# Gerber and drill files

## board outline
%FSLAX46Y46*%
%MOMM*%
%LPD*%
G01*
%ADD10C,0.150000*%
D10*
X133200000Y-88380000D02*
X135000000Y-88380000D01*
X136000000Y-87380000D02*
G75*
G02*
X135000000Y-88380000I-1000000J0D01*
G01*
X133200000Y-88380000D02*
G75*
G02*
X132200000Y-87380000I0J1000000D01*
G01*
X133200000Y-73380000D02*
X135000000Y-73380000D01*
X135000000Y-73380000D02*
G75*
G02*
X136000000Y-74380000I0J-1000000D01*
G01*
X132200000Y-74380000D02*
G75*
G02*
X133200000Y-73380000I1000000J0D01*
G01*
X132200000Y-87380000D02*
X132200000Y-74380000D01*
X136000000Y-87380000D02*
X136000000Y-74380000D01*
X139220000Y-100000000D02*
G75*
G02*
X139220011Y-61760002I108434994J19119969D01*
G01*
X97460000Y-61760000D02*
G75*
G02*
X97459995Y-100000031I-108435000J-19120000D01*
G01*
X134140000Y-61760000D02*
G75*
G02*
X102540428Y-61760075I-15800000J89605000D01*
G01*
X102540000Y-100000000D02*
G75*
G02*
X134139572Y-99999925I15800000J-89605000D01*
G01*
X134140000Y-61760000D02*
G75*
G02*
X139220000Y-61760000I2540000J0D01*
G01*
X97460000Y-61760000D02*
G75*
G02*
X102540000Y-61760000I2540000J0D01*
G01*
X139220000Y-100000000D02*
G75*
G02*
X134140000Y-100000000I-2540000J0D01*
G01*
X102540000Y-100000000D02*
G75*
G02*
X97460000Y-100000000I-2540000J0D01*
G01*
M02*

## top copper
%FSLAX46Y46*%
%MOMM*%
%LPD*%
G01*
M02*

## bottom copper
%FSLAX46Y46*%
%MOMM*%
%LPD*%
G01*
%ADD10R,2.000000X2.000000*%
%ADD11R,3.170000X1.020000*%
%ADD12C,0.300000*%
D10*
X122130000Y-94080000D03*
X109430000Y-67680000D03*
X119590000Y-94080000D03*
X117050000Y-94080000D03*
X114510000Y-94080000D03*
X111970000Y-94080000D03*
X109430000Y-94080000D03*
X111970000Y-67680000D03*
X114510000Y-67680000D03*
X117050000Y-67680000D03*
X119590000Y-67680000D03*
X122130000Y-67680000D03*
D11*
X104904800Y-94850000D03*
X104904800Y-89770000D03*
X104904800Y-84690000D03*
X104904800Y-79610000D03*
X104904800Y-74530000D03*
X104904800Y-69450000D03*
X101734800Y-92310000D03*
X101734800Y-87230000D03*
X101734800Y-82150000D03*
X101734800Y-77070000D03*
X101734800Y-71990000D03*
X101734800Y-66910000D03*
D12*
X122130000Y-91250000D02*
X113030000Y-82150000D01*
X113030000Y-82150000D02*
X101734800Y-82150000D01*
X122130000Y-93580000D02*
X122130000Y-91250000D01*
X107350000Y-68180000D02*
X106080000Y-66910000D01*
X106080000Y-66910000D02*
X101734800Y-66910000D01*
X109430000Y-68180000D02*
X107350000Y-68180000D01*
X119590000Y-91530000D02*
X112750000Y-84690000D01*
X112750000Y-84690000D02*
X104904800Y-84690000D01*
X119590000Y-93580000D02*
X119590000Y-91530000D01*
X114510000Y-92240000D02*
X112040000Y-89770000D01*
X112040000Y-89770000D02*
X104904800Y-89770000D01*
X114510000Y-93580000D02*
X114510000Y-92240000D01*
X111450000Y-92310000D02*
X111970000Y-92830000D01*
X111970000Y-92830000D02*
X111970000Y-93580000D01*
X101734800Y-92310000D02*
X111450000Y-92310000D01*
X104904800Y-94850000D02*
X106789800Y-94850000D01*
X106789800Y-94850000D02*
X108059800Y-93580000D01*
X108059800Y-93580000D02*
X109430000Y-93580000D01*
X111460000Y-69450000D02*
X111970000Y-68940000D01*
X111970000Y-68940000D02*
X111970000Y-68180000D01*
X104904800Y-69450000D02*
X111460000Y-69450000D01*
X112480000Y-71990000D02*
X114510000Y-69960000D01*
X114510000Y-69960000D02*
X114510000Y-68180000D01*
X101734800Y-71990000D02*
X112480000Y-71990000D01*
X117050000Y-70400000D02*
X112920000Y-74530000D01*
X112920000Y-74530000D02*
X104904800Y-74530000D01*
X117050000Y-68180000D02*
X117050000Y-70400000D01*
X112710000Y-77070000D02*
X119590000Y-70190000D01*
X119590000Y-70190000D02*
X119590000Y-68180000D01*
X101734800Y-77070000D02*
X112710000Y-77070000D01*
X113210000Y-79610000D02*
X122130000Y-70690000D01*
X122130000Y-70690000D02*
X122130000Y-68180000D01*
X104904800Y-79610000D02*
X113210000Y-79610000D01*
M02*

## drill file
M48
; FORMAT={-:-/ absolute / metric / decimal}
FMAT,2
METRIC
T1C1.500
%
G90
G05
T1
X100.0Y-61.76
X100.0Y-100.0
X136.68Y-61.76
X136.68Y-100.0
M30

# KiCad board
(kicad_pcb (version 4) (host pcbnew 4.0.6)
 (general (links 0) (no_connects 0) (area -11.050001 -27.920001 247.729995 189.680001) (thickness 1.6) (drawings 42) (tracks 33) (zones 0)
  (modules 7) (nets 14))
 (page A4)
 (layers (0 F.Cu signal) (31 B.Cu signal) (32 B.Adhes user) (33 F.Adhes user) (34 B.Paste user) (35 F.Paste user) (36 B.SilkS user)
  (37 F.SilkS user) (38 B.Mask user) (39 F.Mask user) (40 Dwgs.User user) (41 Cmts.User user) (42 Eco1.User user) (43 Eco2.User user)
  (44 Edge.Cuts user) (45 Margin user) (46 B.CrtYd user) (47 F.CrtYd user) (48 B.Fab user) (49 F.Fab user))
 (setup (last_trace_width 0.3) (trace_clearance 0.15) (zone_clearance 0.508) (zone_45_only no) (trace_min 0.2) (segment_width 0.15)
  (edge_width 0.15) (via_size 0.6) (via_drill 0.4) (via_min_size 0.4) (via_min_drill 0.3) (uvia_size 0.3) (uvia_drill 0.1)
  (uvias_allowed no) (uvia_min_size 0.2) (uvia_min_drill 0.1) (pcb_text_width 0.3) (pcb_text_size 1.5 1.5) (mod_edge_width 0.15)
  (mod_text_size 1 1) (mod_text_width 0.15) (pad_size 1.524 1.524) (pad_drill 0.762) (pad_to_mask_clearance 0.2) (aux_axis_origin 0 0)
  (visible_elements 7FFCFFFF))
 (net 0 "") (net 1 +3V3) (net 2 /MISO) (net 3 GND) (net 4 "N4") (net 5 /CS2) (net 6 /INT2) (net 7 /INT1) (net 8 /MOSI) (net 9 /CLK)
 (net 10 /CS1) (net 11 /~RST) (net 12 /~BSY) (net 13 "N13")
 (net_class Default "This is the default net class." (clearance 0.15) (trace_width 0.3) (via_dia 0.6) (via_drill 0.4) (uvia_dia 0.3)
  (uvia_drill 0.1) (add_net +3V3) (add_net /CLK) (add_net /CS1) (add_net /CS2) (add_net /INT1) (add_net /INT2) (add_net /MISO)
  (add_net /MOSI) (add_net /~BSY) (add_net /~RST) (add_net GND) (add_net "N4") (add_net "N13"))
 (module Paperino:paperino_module (layer B.Cu) (at 118.73 80.88 90)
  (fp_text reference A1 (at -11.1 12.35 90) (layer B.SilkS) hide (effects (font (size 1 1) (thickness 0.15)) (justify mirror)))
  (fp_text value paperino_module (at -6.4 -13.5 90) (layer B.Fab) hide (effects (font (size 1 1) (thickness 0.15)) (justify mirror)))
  (pad 1 smd rect (at -12.7 3.4 90) (size 2 2) (drill (offset -0.5 0)) (layers B.Cu B.Paste B.Mask) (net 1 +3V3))
  (pad 7 smd rect (at 12.7 -9.3 90) (size 2 2) (drill (offset 0.5 0)) (layers B.Cu B.Paste B.Mask) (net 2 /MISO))
  (pad 2 smd rect (at -12.7 0.86 90) (size 2 2) (drill (offset -0.5 0)) (layers B.Cu B.Paste B.Mask) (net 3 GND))
  (pad 3 smd rect (at -12.7 -1.68 90) (size 2 2) (drill (offset -0.5 0)) (layers B.Cu B.Paste B.Mask) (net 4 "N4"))
  (pad 4 smd rect (at -12.7 -4.22 90) (size 2 2) (drill (offset -0.5 0)) (layers B.Cu B.Paste B.Mask) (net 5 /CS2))
  (pad 5 smd rect (at -12.7 -6.76 90) (size 2 2) (drill (offset -0.5 0)) (layers B.Cu B.Paste B.Mask) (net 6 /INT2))
  (pad 6 smd rect (at -12.7 -9.3 90) (size 2 2) (drill (offset -0.5 0)) (layers B.Cu B.Paste B.Mask) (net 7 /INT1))
  (pad 8 smd rect (at 12.7 -6.76 90) (size 2 2) (drill (offset 0.5 0)) (layers B.Cu B.Paste B.Mask) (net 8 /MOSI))
  (pad 9 smd rect (at 12.7 -4.22 90) (size 2 2) (drill (offset 0.5 0)) (layers B.Cu B.Paste B.Mask) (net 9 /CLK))
  (pad 10 smd rect (at 12.7 -1.68 90) (size 2 2) (drill (offset 0.5 0)) (layers B.Cu B.Paste B.Mask) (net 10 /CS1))
  (pad 11 smd rect (at 12.7 0.86 90) (size 2 2) (drill (offset 0.5 0)) (layers B.Cu B.Paste B.Mask) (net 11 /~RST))
  (pad 12 smd rect (at 12.7 3.4 90) (size 2 2) (drill (offset 0.5 0)) (layers B.Cu B.Paste B.Mask) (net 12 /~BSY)))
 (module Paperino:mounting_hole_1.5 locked (layer F.Cu) (at 100 100)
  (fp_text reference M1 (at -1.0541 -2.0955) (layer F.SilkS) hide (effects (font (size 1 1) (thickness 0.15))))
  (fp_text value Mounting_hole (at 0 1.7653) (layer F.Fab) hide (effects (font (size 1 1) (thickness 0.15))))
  (pad "" np_thru_hole circle (at 0 0) (size 1.5 1.5) (drill 1.5) (layers *.Cu *.Mask)))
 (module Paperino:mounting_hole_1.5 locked (layer F.Cu) (at 136.68 100)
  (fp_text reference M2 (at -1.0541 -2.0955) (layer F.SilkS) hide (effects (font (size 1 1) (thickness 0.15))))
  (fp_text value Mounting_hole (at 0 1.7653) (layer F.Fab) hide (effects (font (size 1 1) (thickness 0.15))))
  (pad "" np_thru_hole circle (at 0 0) (size 1.5 1.5) (drill 1.5) (layers *.Cu *.Mask)))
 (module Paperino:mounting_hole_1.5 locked (layer F.Cu) (at 100 61.76)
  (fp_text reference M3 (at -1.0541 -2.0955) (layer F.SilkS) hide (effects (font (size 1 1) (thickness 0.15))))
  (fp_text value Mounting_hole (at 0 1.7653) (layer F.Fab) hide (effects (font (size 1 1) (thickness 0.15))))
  (pad "" np_thru_hole circle (at 0 0) (size 1.5 1.5) (drill 1.5) (layers *.Cu *.Mask)))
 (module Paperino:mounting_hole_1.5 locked (layer F.Cu) (at 136.68 61.76)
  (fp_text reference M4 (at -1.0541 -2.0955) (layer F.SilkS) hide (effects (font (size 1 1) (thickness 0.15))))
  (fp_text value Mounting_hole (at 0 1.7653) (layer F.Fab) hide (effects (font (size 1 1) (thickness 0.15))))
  (pad "" np_thru_hole circle (at 0 0) (size 1.5 1.5) (drill 1.5) (layers *.Cu *.Mask)))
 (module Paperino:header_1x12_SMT (layer B.Cu) (at 103.32 80.88 90)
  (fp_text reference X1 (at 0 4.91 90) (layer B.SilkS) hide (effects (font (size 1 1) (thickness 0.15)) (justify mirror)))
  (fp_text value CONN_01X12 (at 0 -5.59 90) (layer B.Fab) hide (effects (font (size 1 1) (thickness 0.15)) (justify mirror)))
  (pad 1 smd rect (at -13.97 1.5848 90) (size 1.02 3.17) (layers B.Cu B.Paste B.Mask) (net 7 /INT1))
  (pad 3 smd rect (at -8.89 1.5848 90) (size 1.02 3.17) (layers B.Cu B.Paste B.Mask) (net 5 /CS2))
  (pad 5 smd rect (at -3.81 1.5848 90) (size 1.02 3.17) (layers B.Cu B.Paste B.Mask) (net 3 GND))
  (pad 7 smd rect (at 1.27 1.5848 90) (size 1.02 3.17) (layers B.Cu B.Paste B.Mask) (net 12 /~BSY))
  (pad 9 smd rect (at 6.35 1.5848 90) (size 1.02 3.17) (layers B.Cu B.Paste B.Mask) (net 10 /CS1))
  (pad 11 smd rect (at 11.43 1.5848 90) (size 1.02 3.17) (layers B.Cu B.Paste B.Mask) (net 8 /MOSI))
  (pad 2 smd rect (at -11.43 -1.5852 90) (size 1.02 3.17) (layers B.Cu B.Paste B.Mask) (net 6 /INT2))
  (pad 4 smd rect (at -6.35 -1.5852 90) (size 1.02 3.17) (layers B.Cu B.Paste B.Mask) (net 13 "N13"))
  (pad 6 smd rect (at -1.27 -1.5852 90) (size 1.02 3.17) (layers B.Cu B.Paste B.Mask) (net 1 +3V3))
  (pad 8 smd rect (at 3.81 -1.5852 90) (size 1.02 3.17) (layers B.Cu B.Paste B.Mask) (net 11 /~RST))
  (pad 10 smd rect (at 8.89 -1.5852 90) (size 1.02 3.17) (layers B.Cu B.Paste B.Mask) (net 9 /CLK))
  (pad 12 smd rect (at 13.97 -1.5852 90) (size 1.02 3.17) (layers B.Cu B.Paste B.Mask) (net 2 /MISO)))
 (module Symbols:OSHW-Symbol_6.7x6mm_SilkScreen (layer F.Cu) (at 133.66 67.9 90)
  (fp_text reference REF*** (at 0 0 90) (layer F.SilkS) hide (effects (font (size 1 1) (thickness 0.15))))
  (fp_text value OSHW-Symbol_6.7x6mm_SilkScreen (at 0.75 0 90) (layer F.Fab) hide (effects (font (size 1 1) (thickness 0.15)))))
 (gr_line (start 133.2 88.38) (end 135 88.38) (layer Edge.Cuts) (width 0.15))
 (gr_arc (start 135 87.38) (end 136 87.38) (angle 90) (layer Edge.Cuts) (width 0.15))
 (gr_arc (start 133.2 87.38) (end 133.2 88.38) (angle 90) (layer Edge.Cuts) (width 0.15))
 (gr_line (start 133.2 73.38) (end 135 73.38) (layer Edge.Cuts) (width 0.15))
 (gr_arc (start 135 74.38) (end 135 73.38) (angle 90) (layer Edge.Cuts) (width 0.15))
 (gr_arc (start 133.2 74.38) (end 132.2 74.38) (angle 90) (layer Edge.Cuts) (width 0.15))
 (gr_line (start 132.2 87.38) (end 132.2 74.38) (layer Edge.Cuts) (width 0.15))
 (gr_line (start 136 87.38) (end 136 74.38) (layer Edge.Cuts) (width 0.15))
 (gr_arc (start 247.654994 80.880031) (end 139.22 100) (angle 19.9999845) (layer Edge.Cuts) (width 0.15))
 (gr_arc (start -10.975 80.88) (end 97.46 61.76) (angle 20) (layer Edge.Cuts) (width 0.15))
 (gr_arc (start 118.34 -27.845) (end 134.14 61.76) (angle 20) (layer Edge.Cuts) (width 0.15))
 (gr_arc (start 118.34 189.605) (end 102.54 100) (angle 20) (layer Edge.Cuts) (width 0.15))
 (gr_arc (start 136.68 61.76) (end 134.14 61.76) (angle 180) (layer Edge.Cuts) (width 0.15))
 (gr_arc (start 100 61.76) (end 97.46 61.76) (angle 180) (layer Edge.Cuts) (width 0.15))
 (gr_arc (start 136.68 100) (end 139.22 100) (angle 180) (layer Edge.Cuts) (width 0.15))
 (gr_arc (start 100 100) (end 102.54 100) (angle 180) (layer Edge.Cuts) (width 0.15))
 (segment (start 122.13 91.25) (end 113.03 82.15) (width 0.3) (layer B.Cu) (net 1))
 (segment (start 113.03 82.15) (end 101.7348 82.15) (width 0.3) (layer B.Cu) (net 1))
 (segment (start 122.13 93.58) (end 122.13 91.25) (width 0.3) (layer B.Cu) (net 1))
 (segment (start 107.35 68.18) (end 106.08 66.91) (width 0.3) (layer B.Cu) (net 2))
 (segment (start 106.08 66.91) (end 101.7348 66.91) (width 0.3) (layer B.Cu) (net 2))
 (segment (start 109.43 68.18) (end 107.35 68.18) (width 0.3) (layer B.Cu) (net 2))
 (segment (start 119.59 91.53) (end 112.75 84.69) (width 0.3) (layer B.Cu) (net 3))
 (segment (start 112.75 84.69) (end 104.9048 84.69) (width 0.3) (layer B.Cu) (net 3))
 (segment (start 119.59 93.58) (end 119.59 91.53) (width 0.3) (layer B.Cu) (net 3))
 (segment (start 114.51 92.24) (end 112.04 89.77) (width 0.3) (layer B.Cu) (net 5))
 (segment (start 112.04 89.77) (end 104.9048 89.77) (width 0.3) (layer B.Cu) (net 5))
 (segment (start 114.51 93.58) (end 114.51 92.24) (width 0.3) (layer B.Cu) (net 5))
 (segment (start 111.45 92.31) (end 111.97 92.83) (width 0.3) (layer B.Cu) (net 6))
 (segment (start 111.97 92.83) (end 111.97 93.58) (width 0.3) (layer B.Cu) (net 6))
 (segment (start 101.7348 92.31) (end 111.45 92.31) (width 0.3) (layer B.Cu) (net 6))
 (segment (start 104.9048 94.85) (end 106.7898 94.85) (width 0.3) (layer B.Cu) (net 7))
 (segment (start 106.7898 94.85) (end 108.0598 93.58) (width 0.3) (layer B.Cu) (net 7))
 (segment (start 108.0598 93.58) (end 109.43 93.58) (width 0.3) (layer B.Cu) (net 7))
 (segment (start 111.46 69.45) (end 111.97 68.94) (width 0.3) (layer B.Cu) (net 8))
 (segment (start 111.97 68.94) (end 111.97 68.18) (width 0.3) (layer B.Cu) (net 8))
 (segment (start 104.9048 69.45) (end 111.46 69.45) (width 0.3) (layer B.Cu) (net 8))
 (segment (start 112.48 71.99) (end 114.51 69.96) (width 0.3) (layer B.Cu) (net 9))
 (segment (start 114.51 69.96) (end 114.51 68.18) (width 0.3) (layer B.Cu) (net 9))
 (segment (start 101.7348 71.99) (end 112.48 71.99) (width 0.3) (layer B.Cu) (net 9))
 (segment (start 117.05 70.4) (end 112.92 74.53) (width 0.3) (layer B.Cu) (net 10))
 (segment (start 112.92 74.53) (end 104.9048 74.53) (width 0.3) (layer B.Cu) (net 10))
 (segment (start 117.05 68.18) (end 117.05 70.4) (width 0.3) (layer B.Cu) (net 10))
 (segment (start 112.71 77.07) (end 119.59 70.19) (width 0.3) (layer B.Cu) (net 11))
 (segment (start 119.59 70.19) (end 119.59 68.18) (width 0.3) (layer B.Cu) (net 11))
 (segment (start 101.7348 77.07) (end 112.71 77.07) (width 0.3) (layer B.Cu) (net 11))
 (segment (start 113.21 79.61) (end 122.13 70.69) (width 0.3) (layer B.Cu) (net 12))
 (segment (start 122.13 70.69) (end 122.13 68.18) (width 0.3) (layer B.Cu) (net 12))
 (segment (start 104.9048 79.61) (end 113.21 79.61) (width 0.3) (layer B.Cu) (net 12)))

